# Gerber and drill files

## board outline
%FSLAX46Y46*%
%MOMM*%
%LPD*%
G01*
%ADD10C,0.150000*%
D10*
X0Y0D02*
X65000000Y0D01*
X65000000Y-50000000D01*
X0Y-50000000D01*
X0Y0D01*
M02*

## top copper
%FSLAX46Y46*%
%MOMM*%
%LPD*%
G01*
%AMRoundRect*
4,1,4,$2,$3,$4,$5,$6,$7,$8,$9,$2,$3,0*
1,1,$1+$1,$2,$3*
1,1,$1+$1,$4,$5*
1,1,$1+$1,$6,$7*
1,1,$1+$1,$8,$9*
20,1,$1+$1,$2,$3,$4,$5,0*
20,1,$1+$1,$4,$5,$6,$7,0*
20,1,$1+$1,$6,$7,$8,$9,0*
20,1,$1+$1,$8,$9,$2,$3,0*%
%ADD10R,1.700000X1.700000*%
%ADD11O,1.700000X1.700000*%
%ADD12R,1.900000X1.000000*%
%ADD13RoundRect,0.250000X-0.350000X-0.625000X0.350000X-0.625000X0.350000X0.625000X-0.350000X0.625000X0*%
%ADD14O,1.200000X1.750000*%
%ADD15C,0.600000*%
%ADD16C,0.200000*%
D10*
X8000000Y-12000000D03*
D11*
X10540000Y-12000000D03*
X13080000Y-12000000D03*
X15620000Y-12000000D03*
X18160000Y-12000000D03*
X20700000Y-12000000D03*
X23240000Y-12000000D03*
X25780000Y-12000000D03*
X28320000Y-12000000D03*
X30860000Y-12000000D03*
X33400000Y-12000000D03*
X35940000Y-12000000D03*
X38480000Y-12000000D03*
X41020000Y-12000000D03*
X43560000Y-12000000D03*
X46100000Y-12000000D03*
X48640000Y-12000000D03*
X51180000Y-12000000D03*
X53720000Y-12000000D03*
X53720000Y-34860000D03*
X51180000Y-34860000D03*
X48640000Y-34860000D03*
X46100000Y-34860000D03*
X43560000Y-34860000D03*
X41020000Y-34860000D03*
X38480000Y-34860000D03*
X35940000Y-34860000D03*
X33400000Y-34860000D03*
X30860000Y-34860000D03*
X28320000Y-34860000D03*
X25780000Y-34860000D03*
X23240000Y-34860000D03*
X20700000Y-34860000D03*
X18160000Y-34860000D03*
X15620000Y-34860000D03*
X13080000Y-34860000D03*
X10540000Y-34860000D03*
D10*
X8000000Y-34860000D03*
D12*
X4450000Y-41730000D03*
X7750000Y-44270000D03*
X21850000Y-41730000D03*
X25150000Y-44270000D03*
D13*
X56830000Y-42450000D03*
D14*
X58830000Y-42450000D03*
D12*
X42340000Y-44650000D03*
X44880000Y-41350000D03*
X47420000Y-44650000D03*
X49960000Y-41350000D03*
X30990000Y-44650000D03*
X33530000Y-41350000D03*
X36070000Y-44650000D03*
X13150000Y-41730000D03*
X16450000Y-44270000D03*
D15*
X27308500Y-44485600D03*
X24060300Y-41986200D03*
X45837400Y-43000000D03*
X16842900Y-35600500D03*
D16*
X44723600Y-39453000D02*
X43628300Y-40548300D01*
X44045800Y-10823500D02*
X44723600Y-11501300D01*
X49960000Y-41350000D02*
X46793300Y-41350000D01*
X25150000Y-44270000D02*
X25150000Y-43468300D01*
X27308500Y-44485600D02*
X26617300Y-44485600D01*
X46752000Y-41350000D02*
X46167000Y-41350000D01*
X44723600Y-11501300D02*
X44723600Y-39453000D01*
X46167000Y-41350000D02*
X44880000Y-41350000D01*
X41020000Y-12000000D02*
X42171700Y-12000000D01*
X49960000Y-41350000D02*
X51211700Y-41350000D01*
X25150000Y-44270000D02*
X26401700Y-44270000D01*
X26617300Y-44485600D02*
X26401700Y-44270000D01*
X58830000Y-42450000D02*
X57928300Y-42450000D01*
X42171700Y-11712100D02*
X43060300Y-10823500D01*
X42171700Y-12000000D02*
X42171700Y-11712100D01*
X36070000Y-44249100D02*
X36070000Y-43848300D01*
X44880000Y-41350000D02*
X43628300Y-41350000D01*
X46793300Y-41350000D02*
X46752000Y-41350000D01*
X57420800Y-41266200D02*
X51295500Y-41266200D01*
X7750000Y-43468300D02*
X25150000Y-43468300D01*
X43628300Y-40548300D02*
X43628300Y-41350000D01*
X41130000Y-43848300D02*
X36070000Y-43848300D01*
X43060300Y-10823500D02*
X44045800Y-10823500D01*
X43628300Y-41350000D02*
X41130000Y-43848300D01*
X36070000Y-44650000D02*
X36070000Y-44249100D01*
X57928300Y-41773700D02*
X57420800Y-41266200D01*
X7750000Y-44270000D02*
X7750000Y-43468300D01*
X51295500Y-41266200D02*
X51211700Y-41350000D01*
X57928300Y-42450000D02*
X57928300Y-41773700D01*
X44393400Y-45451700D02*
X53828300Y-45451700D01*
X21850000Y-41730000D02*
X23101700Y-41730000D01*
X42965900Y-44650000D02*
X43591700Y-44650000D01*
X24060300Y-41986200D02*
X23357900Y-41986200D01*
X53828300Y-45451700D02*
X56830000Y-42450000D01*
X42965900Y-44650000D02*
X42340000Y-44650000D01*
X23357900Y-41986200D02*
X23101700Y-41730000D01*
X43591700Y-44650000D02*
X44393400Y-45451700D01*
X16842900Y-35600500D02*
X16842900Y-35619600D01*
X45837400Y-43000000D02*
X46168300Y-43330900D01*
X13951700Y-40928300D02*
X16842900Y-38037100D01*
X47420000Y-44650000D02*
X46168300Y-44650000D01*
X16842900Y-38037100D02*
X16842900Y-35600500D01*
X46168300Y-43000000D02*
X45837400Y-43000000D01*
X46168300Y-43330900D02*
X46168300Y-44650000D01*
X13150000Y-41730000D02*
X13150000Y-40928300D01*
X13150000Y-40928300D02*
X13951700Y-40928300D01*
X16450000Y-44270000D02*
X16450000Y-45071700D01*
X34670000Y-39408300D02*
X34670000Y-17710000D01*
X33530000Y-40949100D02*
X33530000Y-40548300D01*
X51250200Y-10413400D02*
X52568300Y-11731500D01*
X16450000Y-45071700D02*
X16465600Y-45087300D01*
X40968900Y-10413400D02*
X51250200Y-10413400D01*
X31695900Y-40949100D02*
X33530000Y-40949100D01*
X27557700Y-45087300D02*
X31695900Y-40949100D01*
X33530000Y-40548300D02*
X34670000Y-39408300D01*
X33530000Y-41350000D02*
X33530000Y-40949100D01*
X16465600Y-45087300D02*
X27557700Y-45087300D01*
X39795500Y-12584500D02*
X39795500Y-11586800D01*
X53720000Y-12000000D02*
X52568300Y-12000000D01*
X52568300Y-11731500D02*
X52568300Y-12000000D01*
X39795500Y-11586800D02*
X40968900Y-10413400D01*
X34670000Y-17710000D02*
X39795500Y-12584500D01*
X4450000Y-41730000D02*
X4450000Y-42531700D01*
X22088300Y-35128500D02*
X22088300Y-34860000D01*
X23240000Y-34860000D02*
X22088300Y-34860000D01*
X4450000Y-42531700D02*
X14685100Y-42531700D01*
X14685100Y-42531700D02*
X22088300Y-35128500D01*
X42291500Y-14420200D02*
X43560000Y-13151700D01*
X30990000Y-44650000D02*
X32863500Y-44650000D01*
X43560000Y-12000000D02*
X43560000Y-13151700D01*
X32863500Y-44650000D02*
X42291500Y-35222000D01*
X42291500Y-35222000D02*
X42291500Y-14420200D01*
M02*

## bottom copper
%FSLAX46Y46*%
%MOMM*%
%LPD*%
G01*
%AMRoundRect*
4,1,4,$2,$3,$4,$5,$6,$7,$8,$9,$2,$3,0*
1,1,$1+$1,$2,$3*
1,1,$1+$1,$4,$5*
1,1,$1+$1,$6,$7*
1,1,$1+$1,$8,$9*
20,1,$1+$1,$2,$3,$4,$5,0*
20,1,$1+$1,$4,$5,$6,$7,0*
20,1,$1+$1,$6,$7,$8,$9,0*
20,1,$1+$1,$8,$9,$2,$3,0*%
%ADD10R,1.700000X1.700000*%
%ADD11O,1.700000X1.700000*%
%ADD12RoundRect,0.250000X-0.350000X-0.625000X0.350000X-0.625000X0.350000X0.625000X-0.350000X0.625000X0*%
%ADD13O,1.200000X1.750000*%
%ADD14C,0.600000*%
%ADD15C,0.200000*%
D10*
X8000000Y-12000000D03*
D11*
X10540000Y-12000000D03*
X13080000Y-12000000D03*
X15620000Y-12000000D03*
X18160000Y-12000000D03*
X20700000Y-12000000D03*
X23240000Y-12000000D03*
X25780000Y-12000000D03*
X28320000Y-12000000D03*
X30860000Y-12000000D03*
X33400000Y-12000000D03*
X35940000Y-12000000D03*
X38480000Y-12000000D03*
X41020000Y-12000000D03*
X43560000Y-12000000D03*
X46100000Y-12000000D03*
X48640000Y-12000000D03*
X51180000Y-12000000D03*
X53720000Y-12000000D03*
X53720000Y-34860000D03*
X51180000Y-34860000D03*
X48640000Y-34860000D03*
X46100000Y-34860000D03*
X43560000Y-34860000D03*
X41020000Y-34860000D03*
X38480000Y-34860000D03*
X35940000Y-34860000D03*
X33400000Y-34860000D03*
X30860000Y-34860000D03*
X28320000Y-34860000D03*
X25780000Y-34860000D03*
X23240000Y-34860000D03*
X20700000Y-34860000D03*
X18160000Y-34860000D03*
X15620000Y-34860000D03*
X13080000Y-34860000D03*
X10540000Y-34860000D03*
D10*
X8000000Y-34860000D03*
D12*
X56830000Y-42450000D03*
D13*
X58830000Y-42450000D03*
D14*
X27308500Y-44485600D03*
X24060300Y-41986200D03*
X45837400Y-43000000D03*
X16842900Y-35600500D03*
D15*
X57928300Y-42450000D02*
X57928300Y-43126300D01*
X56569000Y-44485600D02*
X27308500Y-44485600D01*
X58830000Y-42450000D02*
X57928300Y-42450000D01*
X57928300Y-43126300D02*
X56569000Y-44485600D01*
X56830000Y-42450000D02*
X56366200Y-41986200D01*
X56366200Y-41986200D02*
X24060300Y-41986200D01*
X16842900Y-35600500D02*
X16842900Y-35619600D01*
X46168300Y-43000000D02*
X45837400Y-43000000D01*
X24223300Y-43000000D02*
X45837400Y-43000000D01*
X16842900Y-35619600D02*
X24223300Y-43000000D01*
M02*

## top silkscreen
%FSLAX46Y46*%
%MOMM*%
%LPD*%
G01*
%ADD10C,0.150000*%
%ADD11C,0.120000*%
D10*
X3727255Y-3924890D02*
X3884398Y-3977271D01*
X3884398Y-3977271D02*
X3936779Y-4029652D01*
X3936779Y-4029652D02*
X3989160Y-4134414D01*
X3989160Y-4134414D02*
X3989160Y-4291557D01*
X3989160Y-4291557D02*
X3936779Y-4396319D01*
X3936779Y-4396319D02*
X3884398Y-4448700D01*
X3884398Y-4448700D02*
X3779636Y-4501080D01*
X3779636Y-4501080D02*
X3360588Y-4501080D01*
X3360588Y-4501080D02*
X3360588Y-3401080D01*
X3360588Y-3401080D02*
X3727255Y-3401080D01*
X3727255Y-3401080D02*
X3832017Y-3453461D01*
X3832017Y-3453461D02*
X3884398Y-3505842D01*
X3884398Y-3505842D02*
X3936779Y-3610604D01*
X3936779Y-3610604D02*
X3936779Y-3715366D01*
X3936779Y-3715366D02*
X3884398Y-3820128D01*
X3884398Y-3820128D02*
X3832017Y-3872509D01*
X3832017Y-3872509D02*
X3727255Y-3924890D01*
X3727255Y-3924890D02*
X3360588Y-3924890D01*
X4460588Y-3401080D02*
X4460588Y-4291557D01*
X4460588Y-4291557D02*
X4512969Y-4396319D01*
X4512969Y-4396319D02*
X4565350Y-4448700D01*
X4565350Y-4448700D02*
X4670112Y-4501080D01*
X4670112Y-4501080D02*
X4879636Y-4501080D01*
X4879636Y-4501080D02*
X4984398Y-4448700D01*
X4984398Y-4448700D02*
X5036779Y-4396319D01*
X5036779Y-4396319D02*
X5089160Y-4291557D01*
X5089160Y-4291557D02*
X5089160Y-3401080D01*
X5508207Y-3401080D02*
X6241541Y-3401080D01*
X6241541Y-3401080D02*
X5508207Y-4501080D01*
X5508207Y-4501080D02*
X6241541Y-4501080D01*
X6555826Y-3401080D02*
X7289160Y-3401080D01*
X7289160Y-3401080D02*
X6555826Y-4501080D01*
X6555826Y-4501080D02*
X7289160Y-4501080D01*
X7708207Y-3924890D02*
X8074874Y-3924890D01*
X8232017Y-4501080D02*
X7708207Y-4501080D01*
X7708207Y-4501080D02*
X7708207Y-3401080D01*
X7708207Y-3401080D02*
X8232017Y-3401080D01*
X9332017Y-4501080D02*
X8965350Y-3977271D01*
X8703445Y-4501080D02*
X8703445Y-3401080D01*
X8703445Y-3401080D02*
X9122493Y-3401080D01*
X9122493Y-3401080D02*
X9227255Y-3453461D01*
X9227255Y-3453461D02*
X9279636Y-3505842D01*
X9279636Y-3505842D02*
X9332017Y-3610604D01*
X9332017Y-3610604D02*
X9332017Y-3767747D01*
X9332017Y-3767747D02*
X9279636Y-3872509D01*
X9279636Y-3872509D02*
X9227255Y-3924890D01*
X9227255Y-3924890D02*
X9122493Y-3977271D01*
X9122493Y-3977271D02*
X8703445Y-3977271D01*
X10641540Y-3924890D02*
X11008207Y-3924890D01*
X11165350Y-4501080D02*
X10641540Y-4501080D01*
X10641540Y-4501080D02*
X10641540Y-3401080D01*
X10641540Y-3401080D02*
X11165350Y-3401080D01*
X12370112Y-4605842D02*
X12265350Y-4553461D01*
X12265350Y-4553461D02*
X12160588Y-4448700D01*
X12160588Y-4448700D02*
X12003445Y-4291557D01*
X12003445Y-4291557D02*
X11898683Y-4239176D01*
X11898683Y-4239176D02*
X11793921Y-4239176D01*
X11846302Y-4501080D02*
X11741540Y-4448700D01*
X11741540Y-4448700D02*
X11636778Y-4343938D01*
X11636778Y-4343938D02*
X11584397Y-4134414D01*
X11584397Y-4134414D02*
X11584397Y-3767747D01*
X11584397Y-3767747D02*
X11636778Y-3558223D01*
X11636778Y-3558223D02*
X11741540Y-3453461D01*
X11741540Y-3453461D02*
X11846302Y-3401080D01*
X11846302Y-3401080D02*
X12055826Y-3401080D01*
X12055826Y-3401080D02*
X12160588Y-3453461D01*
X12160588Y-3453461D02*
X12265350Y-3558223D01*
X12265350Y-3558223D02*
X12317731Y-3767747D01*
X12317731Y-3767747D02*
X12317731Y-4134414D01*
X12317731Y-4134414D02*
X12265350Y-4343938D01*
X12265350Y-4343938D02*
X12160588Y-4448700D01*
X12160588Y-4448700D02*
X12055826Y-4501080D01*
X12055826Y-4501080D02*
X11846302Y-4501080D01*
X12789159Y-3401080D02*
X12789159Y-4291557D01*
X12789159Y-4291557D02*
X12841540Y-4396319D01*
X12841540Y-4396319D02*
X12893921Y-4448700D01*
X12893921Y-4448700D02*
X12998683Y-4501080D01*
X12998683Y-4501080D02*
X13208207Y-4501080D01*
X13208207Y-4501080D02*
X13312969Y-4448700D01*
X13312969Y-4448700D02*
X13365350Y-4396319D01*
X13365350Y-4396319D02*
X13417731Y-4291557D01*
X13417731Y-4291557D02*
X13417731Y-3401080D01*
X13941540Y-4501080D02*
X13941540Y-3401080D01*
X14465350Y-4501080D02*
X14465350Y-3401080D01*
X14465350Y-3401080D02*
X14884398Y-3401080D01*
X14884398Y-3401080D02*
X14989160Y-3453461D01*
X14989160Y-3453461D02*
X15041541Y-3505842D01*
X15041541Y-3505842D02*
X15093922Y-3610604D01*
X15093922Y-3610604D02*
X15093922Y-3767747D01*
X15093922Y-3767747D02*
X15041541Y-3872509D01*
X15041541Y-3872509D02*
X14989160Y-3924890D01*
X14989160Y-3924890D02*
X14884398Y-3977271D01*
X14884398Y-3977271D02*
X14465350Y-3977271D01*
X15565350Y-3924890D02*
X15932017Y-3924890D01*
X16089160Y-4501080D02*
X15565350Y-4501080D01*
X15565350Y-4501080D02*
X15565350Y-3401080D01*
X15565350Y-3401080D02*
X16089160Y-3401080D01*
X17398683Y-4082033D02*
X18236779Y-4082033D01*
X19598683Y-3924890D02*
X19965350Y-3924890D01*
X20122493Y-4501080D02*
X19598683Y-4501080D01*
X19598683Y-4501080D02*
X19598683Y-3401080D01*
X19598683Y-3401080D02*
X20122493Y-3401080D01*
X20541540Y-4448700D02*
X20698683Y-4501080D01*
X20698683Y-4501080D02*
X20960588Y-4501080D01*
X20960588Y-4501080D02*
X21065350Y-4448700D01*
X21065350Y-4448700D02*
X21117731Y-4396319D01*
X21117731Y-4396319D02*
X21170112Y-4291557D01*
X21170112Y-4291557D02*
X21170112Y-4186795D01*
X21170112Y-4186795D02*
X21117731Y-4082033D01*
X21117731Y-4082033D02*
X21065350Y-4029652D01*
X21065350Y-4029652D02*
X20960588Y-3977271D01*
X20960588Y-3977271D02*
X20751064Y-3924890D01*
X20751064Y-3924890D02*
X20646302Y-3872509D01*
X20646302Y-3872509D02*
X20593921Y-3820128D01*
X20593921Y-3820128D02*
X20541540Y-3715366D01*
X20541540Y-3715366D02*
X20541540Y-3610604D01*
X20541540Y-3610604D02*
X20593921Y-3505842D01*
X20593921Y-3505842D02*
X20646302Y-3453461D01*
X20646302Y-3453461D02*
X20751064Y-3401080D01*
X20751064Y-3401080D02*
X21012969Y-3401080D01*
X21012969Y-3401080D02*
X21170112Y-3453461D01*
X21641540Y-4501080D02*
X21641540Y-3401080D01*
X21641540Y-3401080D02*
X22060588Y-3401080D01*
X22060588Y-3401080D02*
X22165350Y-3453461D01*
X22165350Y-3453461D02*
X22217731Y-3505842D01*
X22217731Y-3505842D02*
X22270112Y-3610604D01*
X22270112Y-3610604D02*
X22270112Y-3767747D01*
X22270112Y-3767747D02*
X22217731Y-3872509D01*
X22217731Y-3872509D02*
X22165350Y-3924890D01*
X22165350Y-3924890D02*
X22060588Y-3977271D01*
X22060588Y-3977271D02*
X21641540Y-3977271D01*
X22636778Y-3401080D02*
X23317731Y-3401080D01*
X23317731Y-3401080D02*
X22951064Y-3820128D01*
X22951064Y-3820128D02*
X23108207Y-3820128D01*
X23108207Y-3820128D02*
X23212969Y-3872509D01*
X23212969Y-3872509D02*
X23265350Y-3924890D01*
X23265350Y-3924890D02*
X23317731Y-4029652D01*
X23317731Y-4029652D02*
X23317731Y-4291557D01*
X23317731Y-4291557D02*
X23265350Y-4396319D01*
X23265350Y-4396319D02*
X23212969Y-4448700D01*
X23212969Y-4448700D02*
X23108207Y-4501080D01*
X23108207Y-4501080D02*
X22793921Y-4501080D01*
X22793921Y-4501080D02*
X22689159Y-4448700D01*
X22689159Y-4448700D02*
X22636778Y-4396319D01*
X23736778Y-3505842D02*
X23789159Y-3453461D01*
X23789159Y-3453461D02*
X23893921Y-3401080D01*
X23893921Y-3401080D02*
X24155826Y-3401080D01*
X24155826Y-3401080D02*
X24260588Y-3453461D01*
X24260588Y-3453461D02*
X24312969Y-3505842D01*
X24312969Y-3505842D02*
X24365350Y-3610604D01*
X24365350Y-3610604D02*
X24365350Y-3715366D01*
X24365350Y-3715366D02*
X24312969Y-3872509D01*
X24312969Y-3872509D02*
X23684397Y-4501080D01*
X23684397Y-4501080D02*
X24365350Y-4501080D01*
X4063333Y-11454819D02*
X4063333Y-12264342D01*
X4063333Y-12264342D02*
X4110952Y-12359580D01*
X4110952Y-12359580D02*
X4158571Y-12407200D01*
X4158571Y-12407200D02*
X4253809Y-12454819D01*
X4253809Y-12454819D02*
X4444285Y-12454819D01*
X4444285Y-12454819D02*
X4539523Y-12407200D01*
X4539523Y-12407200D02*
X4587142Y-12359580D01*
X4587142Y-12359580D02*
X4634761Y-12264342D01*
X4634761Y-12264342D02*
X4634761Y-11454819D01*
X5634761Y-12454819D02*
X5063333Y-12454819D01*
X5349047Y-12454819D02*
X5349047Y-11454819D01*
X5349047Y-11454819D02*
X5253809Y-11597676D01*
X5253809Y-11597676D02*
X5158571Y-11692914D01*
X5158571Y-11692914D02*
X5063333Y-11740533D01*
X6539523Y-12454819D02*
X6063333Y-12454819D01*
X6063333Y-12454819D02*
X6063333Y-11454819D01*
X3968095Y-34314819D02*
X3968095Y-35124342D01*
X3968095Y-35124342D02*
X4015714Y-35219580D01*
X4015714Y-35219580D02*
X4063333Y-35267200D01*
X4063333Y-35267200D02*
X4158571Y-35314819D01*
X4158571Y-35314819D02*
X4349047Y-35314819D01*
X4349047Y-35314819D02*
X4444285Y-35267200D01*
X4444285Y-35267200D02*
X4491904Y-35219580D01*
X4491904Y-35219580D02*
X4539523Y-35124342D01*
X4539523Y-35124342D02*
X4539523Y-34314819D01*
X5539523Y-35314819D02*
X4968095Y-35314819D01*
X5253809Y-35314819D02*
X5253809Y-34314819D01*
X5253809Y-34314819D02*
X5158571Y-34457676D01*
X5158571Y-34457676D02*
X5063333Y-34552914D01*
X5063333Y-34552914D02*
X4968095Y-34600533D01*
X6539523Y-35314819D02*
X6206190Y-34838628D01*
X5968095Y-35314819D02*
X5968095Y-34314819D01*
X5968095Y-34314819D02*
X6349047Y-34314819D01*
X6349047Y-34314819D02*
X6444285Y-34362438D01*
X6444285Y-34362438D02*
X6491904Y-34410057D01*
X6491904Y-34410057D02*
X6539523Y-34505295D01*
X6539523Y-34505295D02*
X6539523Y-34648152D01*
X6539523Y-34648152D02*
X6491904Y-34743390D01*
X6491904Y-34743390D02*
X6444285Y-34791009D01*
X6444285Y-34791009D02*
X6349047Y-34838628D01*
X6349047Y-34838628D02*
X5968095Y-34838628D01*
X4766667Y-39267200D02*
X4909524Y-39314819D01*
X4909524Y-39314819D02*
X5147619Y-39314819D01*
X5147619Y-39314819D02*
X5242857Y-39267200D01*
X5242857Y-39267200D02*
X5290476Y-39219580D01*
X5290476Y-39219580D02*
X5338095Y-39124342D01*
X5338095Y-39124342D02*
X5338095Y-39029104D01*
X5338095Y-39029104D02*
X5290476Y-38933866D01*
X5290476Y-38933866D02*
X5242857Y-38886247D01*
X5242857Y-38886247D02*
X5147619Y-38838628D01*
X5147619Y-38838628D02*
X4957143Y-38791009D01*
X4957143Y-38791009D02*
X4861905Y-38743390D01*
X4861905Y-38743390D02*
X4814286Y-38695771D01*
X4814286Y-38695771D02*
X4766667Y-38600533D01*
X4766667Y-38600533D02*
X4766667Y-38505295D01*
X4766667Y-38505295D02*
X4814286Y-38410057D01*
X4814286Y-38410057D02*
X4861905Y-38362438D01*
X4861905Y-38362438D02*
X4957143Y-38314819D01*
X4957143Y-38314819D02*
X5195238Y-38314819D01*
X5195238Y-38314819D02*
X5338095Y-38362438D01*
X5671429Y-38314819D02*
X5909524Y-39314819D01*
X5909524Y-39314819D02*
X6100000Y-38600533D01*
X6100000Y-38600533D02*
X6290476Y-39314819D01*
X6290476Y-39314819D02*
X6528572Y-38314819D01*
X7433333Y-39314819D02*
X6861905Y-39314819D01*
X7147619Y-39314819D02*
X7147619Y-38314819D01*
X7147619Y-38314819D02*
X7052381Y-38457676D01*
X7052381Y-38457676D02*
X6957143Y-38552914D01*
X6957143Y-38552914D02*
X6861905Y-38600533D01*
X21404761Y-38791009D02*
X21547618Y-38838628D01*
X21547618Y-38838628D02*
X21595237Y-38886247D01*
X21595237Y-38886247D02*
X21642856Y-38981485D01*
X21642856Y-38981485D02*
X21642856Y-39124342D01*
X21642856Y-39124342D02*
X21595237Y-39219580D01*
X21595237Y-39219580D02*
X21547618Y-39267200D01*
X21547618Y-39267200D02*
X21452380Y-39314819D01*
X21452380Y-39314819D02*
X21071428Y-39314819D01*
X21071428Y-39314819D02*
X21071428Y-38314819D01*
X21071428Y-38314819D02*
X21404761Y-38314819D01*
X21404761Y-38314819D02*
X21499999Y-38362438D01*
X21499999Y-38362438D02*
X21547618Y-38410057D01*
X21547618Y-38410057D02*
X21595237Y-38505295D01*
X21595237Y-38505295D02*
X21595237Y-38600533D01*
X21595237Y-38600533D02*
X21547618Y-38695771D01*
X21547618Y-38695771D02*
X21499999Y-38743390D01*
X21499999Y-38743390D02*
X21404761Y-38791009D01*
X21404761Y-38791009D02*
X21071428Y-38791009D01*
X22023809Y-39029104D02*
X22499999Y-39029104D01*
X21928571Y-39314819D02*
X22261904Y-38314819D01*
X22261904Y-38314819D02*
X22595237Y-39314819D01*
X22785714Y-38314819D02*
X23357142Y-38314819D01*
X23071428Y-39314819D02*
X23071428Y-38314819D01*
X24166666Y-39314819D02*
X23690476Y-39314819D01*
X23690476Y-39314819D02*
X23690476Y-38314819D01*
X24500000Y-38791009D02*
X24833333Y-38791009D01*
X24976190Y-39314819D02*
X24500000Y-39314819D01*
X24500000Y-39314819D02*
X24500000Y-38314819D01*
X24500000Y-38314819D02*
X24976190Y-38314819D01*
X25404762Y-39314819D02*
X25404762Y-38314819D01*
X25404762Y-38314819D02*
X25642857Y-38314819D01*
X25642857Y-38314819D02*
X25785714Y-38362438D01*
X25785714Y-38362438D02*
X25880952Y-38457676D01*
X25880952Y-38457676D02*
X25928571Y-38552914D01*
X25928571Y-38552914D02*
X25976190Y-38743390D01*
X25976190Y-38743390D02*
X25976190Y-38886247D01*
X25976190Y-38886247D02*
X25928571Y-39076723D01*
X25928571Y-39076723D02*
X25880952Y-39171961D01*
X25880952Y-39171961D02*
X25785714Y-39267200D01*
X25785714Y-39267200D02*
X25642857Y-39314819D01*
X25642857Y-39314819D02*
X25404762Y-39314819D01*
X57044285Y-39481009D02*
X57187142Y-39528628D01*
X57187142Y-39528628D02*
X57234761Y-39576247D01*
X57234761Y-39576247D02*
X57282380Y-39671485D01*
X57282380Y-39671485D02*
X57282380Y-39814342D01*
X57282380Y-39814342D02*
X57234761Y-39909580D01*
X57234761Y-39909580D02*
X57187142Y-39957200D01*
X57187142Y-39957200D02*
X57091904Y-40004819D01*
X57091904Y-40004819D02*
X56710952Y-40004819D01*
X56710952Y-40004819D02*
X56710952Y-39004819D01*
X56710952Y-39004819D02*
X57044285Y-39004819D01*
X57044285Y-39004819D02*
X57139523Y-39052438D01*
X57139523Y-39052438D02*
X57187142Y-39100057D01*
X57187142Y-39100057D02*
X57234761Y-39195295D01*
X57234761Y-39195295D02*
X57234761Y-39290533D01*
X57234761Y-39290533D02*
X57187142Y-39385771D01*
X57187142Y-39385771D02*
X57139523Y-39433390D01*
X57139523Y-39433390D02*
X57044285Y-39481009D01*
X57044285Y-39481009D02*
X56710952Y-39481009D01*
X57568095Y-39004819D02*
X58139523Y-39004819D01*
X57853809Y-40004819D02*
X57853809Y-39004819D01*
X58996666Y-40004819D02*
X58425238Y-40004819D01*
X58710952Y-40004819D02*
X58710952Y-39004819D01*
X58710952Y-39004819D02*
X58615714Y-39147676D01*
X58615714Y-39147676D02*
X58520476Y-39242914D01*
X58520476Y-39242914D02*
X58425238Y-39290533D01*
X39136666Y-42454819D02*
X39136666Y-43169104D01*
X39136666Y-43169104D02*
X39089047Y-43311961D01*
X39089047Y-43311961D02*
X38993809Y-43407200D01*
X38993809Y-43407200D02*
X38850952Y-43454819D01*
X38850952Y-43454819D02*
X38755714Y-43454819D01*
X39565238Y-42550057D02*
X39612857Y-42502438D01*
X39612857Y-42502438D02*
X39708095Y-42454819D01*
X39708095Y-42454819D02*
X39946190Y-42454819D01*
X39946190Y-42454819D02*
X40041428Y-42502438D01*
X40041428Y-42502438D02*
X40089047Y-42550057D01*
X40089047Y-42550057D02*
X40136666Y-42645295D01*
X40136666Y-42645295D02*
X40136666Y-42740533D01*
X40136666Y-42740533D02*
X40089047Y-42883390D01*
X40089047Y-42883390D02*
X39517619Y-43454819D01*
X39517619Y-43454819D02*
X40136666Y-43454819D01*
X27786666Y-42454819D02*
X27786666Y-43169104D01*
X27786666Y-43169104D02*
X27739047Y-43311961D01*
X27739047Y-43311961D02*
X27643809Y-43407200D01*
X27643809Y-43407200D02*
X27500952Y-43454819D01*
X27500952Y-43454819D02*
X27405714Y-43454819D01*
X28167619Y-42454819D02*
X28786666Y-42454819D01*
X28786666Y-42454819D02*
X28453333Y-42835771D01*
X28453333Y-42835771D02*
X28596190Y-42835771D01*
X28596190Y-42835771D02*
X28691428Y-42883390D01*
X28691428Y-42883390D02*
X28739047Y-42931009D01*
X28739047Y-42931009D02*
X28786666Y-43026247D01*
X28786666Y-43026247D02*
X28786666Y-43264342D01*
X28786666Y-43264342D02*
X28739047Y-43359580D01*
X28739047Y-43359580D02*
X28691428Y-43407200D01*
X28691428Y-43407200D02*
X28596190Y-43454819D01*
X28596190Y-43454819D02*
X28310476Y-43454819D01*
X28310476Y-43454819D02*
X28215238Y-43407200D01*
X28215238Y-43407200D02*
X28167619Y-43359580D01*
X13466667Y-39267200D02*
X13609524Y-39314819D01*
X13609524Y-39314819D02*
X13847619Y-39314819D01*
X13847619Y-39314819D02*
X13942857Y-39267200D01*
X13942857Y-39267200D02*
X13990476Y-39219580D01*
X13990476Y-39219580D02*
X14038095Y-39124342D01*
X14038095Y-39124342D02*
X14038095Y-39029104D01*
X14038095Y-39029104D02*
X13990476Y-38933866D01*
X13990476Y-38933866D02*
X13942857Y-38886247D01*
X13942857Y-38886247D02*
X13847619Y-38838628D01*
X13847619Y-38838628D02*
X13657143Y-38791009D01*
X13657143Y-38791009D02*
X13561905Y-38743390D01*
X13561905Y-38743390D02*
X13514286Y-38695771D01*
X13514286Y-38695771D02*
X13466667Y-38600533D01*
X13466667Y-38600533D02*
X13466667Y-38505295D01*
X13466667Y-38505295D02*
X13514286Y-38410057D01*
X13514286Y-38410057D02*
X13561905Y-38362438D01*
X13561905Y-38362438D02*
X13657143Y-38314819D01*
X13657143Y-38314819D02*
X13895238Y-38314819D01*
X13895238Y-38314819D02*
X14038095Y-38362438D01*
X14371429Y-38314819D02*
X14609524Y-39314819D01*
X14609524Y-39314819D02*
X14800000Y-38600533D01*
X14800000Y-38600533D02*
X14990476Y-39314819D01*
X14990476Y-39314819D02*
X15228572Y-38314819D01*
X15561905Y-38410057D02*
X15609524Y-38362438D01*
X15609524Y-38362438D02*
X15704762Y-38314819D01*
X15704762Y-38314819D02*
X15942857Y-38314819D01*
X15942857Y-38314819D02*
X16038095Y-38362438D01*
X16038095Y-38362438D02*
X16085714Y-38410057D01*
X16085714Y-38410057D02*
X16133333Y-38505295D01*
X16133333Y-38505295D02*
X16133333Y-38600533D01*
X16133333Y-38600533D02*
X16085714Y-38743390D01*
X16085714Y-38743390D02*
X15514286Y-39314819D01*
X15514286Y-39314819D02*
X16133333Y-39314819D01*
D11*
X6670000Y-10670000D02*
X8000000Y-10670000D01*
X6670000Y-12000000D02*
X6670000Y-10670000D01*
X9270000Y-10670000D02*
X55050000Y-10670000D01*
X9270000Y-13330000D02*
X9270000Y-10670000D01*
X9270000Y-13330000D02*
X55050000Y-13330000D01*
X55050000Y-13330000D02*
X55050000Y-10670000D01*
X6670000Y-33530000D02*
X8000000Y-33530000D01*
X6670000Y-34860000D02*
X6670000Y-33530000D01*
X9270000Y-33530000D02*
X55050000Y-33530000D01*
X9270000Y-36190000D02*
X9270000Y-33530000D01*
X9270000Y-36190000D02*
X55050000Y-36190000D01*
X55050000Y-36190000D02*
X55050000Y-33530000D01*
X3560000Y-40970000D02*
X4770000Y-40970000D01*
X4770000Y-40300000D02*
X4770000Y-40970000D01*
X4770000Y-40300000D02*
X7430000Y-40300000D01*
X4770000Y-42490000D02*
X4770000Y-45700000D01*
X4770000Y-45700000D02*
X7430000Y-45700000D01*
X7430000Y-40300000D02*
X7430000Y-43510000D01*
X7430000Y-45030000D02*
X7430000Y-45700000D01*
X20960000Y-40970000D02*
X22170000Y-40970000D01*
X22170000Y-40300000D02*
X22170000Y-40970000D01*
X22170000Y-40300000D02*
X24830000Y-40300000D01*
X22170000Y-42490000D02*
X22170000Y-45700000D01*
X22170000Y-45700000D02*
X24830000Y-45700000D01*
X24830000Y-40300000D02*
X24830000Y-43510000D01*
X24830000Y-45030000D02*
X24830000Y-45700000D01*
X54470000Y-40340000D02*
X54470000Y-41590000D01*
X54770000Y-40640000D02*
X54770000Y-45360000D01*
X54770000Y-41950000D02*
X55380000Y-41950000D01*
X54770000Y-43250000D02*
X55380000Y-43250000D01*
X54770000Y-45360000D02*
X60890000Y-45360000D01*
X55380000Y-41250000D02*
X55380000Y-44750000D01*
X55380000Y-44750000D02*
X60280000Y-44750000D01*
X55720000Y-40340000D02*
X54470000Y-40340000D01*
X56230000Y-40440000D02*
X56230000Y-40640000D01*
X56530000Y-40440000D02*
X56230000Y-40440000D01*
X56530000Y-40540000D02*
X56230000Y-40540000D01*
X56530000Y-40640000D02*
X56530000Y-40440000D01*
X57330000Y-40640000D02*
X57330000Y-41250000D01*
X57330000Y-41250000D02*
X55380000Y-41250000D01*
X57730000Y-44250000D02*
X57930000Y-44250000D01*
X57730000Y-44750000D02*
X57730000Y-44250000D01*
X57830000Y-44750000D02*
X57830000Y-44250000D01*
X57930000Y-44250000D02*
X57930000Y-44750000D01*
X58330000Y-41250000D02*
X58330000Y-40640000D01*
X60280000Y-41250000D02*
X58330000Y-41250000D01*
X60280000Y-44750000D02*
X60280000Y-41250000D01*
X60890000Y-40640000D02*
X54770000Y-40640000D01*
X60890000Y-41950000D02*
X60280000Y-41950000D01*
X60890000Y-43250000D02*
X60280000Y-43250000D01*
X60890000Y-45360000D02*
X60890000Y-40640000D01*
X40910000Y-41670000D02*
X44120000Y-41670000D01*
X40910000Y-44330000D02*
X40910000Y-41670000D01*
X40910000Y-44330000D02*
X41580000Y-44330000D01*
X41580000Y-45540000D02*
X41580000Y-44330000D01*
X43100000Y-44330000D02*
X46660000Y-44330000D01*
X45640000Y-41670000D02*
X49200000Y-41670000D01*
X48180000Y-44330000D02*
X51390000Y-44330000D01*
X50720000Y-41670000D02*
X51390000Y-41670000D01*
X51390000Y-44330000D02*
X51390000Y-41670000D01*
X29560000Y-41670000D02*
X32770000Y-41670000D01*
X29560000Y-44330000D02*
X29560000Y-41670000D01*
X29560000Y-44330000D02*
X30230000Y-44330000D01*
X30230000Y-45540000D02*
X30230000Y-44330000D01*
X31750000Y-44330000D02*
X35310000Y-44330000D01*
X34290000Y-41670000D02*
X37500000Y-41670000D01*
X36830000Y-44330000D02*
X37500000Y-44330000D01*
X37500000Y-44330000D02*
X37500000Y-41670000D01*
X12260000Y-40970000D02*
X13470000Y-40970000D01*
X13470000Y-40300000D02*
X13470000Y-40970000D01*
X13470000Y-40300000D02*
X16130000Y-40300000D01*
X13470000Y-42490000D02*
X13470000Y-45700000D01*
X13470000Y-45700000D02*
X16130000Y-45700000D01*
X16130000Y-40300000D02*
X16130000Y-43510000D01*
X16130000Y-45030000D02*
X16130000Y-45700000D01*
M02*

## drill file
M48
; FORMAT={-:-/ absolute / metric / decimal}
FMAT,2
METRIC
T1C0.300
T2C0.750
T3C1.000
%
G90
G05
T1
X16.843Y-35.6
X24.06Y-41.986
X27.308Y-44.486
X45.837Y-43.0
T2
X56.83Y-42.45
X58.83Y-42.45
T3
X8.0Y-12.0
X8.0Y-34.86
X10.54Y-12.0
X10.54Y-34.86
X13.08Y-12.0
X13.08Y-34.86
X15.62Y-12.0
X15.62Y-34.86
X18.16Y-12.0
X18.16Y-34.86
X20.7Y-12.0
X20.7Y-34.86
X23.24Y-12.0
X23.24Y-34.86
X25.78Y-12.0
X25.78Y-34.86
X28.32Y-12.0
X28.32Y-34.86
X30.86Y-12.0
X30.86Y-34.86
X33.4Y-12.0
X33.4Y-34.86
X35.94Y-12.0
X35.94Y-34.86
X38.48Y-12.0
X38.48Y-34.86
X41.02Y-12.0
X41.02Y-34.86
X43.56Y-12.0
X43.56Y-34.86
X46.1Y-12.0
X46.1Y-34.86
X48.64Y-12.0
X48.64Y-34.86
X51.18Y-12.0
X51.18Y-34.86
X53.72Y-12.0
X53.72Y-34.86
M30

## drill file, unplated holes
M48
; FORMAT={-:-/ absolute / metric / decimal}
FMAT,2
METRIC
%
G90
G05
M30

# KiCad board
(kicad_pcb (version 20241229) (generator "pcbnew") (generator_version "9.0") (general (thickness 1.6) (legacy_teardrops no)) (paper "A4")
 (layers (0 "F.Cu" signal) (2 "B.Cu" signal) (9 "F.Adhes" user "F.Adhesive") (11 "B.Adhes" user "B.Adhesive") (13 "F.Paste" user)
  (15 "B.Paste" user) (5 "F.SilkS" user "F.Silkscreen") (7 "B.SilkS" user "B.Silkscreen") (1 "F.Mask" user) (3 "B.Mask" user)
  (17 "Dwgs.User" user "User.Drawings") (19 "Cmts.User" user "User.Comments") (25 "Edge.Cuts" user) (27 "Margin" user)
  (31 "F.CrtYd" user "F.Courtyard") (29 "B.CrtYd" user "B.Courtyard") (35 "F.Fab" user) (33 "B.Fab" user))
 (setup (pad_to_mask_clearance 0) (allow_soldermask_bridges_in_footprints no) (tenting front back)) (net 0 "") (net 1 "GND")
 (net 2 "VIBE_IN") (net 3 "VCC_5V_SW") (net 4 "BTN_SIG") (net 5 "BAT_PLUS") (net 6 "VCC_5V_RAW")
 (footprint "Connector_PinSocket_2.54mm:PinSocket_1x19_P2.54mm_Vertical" (layer "F.Cu") (at 8 12 90)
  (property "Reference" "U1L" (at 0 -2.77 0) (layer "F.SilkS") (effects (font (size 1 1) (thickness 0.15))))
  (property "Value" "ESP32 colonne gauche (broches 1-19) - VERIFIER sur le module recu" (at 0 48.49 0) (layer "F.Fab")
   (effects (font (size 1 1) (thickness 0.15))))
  (fp_line (start 1.33 -1.33) (end 1.33 0) (stroke (width 0.12) (type solid)) (layer "F.SilkS"))
  (fp_line (start 0 -1.33) (end 1.33 -1.33) (stroke (width 0.12) (type solid)) (layer "F.SilkS"))
  (fp_line (start 1.33 1.27) (end 1.33 47.05) (stroke (width 0.12) (type solid)) (layer "F.SilkS"))
  (fp_line (start -1.33 1.27) (end 1.33 1.27) (stroke (width 0.12) (type solid)) (layer "F.SilkS"))
  (fp_line (start -1.33 1.27) (end -1.33 47.05) (stroke (width 0.12) (type solid)) (layer "F.SilkS"))
  (fp_line (start -1.33 47.05) (end 1.33 47.05) (stroke (width 0.12) (type solid)) (layer "F.SilkS"))
  (pad "1" thru_hole rect (at 0 0) (size 1.7 1.7) (drill 1) (layers "*.Cu" "*.Mask") (remove_unused_layers no))
  (pad "2" thru_hole oval (at 0 2.54) (size 1.7 1.7) (drill 1) (layers "*.Cu" "*.Mask") (remove_unused_layers no))
  (pad "3" thru_hole oval (at 0 5.08) (size 1.7 1.7) (drill 1) (layers "*.Cu" "*.Mask") (remove_unused_layers no))
  (pad "4" thru_hole oval (at 0 7.62) (size 1.7 1.7) (drill 1) (layers "*.Cu" "*.Mask") (remove_unused_layers no))
  (pad "5" thru_hole oval (at 0 10.16) (size 1.7 1.7) (drill 1) (layers "*.Cu" "*.Mask") (remove_unused_layers no))
  (pad "6" thru_hole oval (at 0 12.7) (size 1.7 1.7) (drill 1) (layers "*.Cu" "*.Mask") (remove_unused_layers no))
  (pad "7" thru_hole oval (at 0 15.24) (size 1.7 1.7) (drill 1) (layers "*.Cu" "*.Mask") (remove_unused_layers no))
  (pad "8" thru_hole oval (at 0 17.78) (size 1.7 1.7) (drill 1) (layers "*.Cu" "*.Mask") (remove_unused_layers no))
  (pad "9" thru_hole oval (at 0 20.32) (size 1.7 1.7) (drill 1) (layers "*.Cu" "*.Mask") (remove_unused_layers no))
  (pad "10" thru_hole oval (at 0 22.86) (size 1.7 1.7) (drill 1) (layers "*.Cu" "*.Mask") (remove_unused_layers no))
  (pad "11" thru_hole oval (at 0 25.4) (size 1.7 1.7) (drill 1) (layers "*.Cu" "*.Mask") (remove_unused_layers no))
  (pad "12" thru_hole oval (at 0 27.94) (size 1.7 1.7) (drill 1) (layers "*.Cu" "*.Mask") (remove_unused_layers no))
  (pad "13" thru_hole oval (at 0 30.48) (size 1.7 1.7) (drill 1) (layers "*.Cu" "*.Mask") (remove_unused_layers no))
  (pad "14" thru_hole oval (at 0 33.02) (size 1.7 1.7) (drill 1) (layers "*.Cu" "*.Mask") (remove_unused_layers no) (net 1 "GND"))
  (pad "15" thru_hole oval (at 0 35.56) (size 1.7 1.7) (drill 1) (layers "*.Cu" "*.Mask") (remove_unused_layers no) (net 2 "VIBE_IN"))
  (pad "16" thru_hole oval (at 0 38.1) (size 1.7 1.7) (drill 1) (layers "*.Cu" "*.Mask") (remove_unused_layers no))
  (pad "17" thru_hole oval (at 0 40.64) (size 1.7 1.7) (drill 1) (layers "*.Cu" "*.Mask") (remove_unused_layers no))
  (pad "18" thru_hole oval (at 0 43.18) (size 1.7 1.7) (drill 1) (layers "*.Cu" "*.Mask") (remove_unused_layers no))
  (pad "19" thru_hole oval (at 0 45.72) (size 1.7 1.7) (drill 1) (layers "*.Cu" "*.Mask") (remove_unused_layers no) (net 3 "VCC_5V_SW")))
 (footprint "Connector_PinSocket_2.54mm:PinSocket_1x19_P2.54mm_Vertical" (layer "F.Cu") (at 8 34.86 90)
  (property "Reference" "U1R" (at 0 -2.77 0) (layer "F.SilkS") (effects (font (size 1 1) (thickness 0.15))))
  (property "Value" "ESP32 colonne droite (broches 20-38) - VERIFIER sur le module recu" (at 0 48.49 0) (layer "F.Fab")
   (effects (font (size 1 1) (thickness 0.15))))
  (fp_line (start 1.33 -1.33) (end 1.33 0) (stroke (width 0.12) (type solid)) (layer "F.SilkS"))
  (fp_line (start 0 -1.33) (end 1.33 -1.33) (stroke (width 0.12) (type solid)) (layer "F.SilkS"))
  (fp_line (start 1.33 1.27) (end 1.33 47.05) (stroke (width 0.12) (type solid)) (layer "F.SilkS"))
  (fp_line (start -1.33 1.27) (end 1.33 1.27) (stroke (width 0.12) (type solid)) (layer "F.SilkS"))
  (fp_line (start -1.33 1.27) (end -1.33 47.05) (stroke (width 0.12) (type solid)) (layer "F.SilkS"))
  (fp_line (start -1.33 47.05) (end 1.33 47.05) (stroke (width 0.12) (type solid)) (layer "F.SilkS"))
  (pad "20" thru_hole oval (at 0 45.72) (size 1.7 1.7) (drill 1) (layers "*.Cu" "*.Mask") (remove_unused_layers no))
  (pad "21" thru_hole oval (at 0 43.18) (size 1.7 1.7) (drill 1) (layers "*.Cu" "*.Mask") (remove_unused_layers no))
  (pad "22" thru_hole oval (at 0 40.64) (size 1.7 1.7) (drill 1) (layers "*.Cu" "*.Mask") (remove_unused_layers no))
  (pad "23" thru_hole oval (at 0 38.1) (size 1.7 1.7) (drill 1) (layers "*.Cu" "*.Mask") (remove_unused_layers no))
  (pad "24" thru_hole oval (at 0 35.56) (size 1.7 1.7) (drill 1) (layers "*.Cu" "*.Mask") (remove_unused_layers no))
  (pad "25" thru_hole oval (at 0 33.02) (size 1.7 1.7) (drill 1) (layers "*.Cu" "*.Mask") (remove_unused_layers no))
  (pad "26" thru_hole oval (at 0 30.48) (size 1.7 1.7) (drill 1) (layers "*.Cu" "*.Mask") (remove_unused_layers no))
  (pad "27" thru_hole oval (at 0 27.94) (size 1.7 1.7) (drill 1) (layers "*.Cu" "*.Mask") (remove_unused_layers no))
  (pad "28" thru_hole oval (at 0 25.4) (size 1.7 1.7) (drill 1) (layers "*.Cu" "*.Mask") (remove_unused_layers no))
  (pad "29" thru_hole oval (at 0 22.86) (size 1.7 1.7) (drill 1) (layers "*.Cu" "*.Mask") (remove_unused_layers no))
  (pad "30" thru_hole oval (at 0 20.32) (size 1.7 1.7) (drill 1) (layers "*.Cu" "*.Mask") (remove_unused_layers no))
  (pad "31" thru_hole oval (at 0 17.78) (size 1.7 1.7) (drill 1) (layers "*.Cu" "*.Mask") (remove_unused_layers no))
  (pad "32" thru_hole oval (at 0 15.24) (size 1.7 1.7) (drill 1) (layers "*.Cu" "*.Mask") (remove_unused_layers no) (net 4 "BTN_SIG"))
  (pad "33" thru_hole oval (at 0 12.7) (size 1.7 1.7) (drill 1) (layers "*.Cu" "*.Mask") (remove_unused_layers no))
  (pad "34" thru_hole oval (at 0 10.16) (size 1.7 1.7) (drill 1) (layers "*.Cu" "*.Mask") (remove_unused_layers no))
  (pad "35" thru_hole oval (at 0 7.62) (size 1.7 1.7) (drill 1) (layers "*.Cu" "*.Mask") (remove_unused_layers no))
  (pad "36" thru_hole oval (at 0 5.08) (size 1.7 1.7) (drill 1) (layers "*.Cu" "*.Mask") (remove_unused_layers no))
  (pad "37" thru_hole oval (at 0 2.54) (size 1.7 1.7) (drill 1) (layers "*.Cu" "*.Mask") (remove_unused_layers no))
  (pad "38" thru_hole rect (at 0 0) (size 1.7 1.7) (drill 1) (layers "*.Cu" "*.Mask") (remove_unused_layers no)))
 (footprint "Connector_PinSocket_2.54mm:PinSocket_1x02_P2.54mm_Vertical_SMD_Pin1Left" (layer "F.Cu") (at 6.1 43)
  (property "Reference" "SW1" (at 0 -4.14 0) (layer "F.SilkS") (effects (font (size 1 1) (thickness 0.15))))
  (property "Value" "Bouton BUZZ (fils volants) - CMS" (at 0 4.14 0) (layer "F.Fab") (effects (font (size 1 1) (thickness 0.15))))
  (fp_line (start -2.54 -2.03) (end -1.33 -2.03) (stroke (width 0.12) (type solid)) (layer "F.SilkS"))
  (fp_line (start -1.33 -2.7) (end -1.33 -2.03) (stroke (width 0.12) (type solid)) (layer "F.SilkS"))
  (fp_line (start -1.33 -2.7) (end 1.33 -2.7) (stroke (width 0.12) (type solid)) (layer "F.SilkS"))
  (fp_line (start -1.33 -0.51) (end -1.33 2.7) (stroke (width 0.12) (type solid)) (layer "F.SilkS"))
  (fp_line (start -1.33 2.7) (end 1.33 2.7) (stroke (width 0.12) (type solid)) (layer "F.SilkS"))
  (fp_line (start 1.33 -2.7) (end 1.33 0.51) (stroke (width 0.12) (type solid)) (layer "F.SilkS"))
  (fp_line (start 1.33 2.03) (end 1.33 2.7) (stroke (width 0.12) (type solid)) (layer "F.SilkS"))
  (pad "1" smd rect (at -1.65 -1.27) (size 1.9 1) (layers "F.Cu" "F.Mask" "F.Paste") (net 4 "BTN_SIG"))
  (pad "2" smd rect (at 1.65 1.27) (size 1.9 1) (layers "F.Cu" "F.Mask" "F.Paste") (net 1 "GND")))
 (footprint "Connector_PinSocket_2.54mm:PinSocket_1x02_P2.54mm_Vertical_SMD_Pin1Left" (layer "F.Cu") (at 23.5 43)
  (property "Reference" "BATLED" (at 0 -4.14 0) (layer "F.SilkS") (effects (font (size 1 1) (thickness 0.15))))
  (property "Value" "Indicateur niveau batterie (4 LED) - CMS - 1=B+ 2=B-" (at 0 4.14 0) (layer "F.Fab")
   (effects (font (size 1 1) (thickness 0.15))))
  (fp_line (start -2.54 -2.03) (end -1.33 -2.03) (stroke (width 0.12) (type solid)) (layer "F.SilkS"))
  (fp_line (start -1.33 -2.7) (end -1.33 -2.03) (stroke (width 0.12) (type solid)) (layer "F.SilkS"))
  (fp_line (start -1.33 -2.7) (end 1.33 -2.7) (stroke (width 0.12) (type solid)) (layer "F.SilkS"))
  (fp_line (start -1.33 -0.51) (end -1.33 2.7) (stroke (width 0.12) (type solid)) (layer "F.SilkS"))
  (fp_line (start -1.33 2.7) (end 1.33 2.7) (stroke (width 0.12) (type solid)) (layer "F.SilkS"))
  (fp_line (start 1.33 -2.7) (end 1.33 0.51) (stroke (width 0.12) (type solid)) (layer "F.SilkS"))
  (fp_line (start 1.33 2.03) (end 1.33 2.7) (stroke (width 0.12) (type solid)) (layer "F.SilkS"))
  (pad "1" smd rect (at -1.65 -1.27) (size 1.9 1) (layers "F.Cu" "F.Mask" "F.Paste") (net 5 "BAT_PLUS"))
  (pad "2" smd rect (at 1.65 1.27) (size 1.9 1) (layers "F.Cu" "F.Mask" "F.Paste") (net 1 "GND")))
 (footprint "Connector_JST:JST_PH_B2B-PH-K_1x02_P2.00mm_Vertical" (layer "F.Cu") (at 56.83 42.45)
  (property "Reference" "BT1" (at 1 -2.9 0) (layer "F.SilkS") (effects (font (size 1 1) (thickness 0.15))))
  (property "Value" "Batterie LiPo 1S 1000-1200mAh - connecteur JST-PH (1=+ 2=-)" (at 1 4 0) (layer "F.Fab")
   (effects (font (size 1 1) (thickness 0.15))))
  (fp_line (start -2.36 -2.11) (end -2.36 -0.86) (stroke (width 0.12) (type solid)) (layer "F.SilkS"))
  (fp_line (start -2.06 -1.81) (end -2.06 2.91) (stroke (width 0.12) (type solid)) (layer "F.SilkS"))
  (fp_line (start -2.06 -0.5) (end -1.45 -0.5) (stroke (width 0.12) (type solid)) (layer "F.SilkS"))
  (fp_line (start -2.06 0.8) (end -1.45 0.8) (stroke (width 0.12) (type solid)) (layer "F.SilkS"))
  (fp_line (start -2.06 2.91) (end 4.06 2.91) (stroke (width 0.12) (type solid)) (layer "F.SilkS"))
  (fp_line (start -1.45 -1.2) (end -1.45 2.3) (stroke (width 0.12) (type solid)) (layer "F.SilkS"))
  (fp_line (start -1.45 2.3) (end 3.45 2.3) (stroke (width 0.12) (type solid)) (layer "F.SilkS"))
  (fp_line (start -1.11 -2.11) (end -2.36 -2.11) (stroke (width 0.12) (type solid)) (layer "F.SilkS"))
  (fp_line (start -0.6 -2.01) (end -0.6 -1.81) (stroke (width 0.12) (type solid)) (layer "F.SilkS"))
  (fp_line (start -0.3 -2.01) (end -0.6 -2.01) (stroke (width 0.12) (type solid)) (layer "F.SilkS"))
  (fp_line (start -0.3 -1.91) (end -0.6 -1.91) (stroke (width 0.12) (type solid)) (layer "F.SilkS"))
  (fp_line (start -0.3 -1.81) (end -0.3 -2.01) (stroke (width 0.12) (type solid)) (layer "F.SilkS"))
  (fp_line (start 0.5 -1.81) (end 0.5 -1.2) (stroke (width 0.12) (type solid)) (layer "F.SilkS"))
  (fp_line (start 0.5 -1.2) (end -1.45 -1.2) (stroke (width 0.12) (type solid)) (layer "F.SilkS"))
  (fp_line (start 0.9 1.8) (end 1.1 1.8) (stroke (width 0.12) (type solid)) (layer "F.SilkS"))
  (fp_line (start 0.9 2.3) (end 0.9 1.8) (stroke (width 0.12) (type solid)) (layer "F.SilkS"))
  (fp_line (start 1 2.3) (end 1 1.8) (stroke (width 0.12) (type solid)) (layer "F.SilkS"))
  (fp_line (start 1.1 1.8) (end 1.1 2.3) (stroke (width 0.12) (type solid)) (layer "F.SilkS"))
  (fp_line (start 1.5 -1.2) (end 1.5 -1.81) (stroke (width 0.12) (type solid)) (layer "F.SilkS"))
  (fp_line (start 3.45 -1.2) (end 1.5 -1.2) (stroke (width 0.12) (type solid)) (layer "F.SilkS"))
  (fp_line (start 3.45 2.3) (end 3.45 -1.2) (stroke (width 0.12) (type solid)) (layer "F.SilkS"))
  (fp_line (start 4.06 -1.81) (end -2.06 -1.81) (stroke (width 0.12) (type solid)) (layer "F.SilkS"))
  (fp_line (start 4.06 -0.5) (end 3.45 -0.5) (stroke (width 0.12) (type solid)) (layer "F.SilkS"))
  (fp_line (start 4.06 0.8) (end 3.45 0.8) (stroke (width 0.12) (type solid)) (layer "F.SilkS"))
  (fp_line (start 4.06 2.91) (end 4.06 -1.81) (stroke (width 0.12) (type solid)) (layer "F.SilkS"))
  (pad "1" thru_hole roundrect (at 0 0) (size 1.2 1.75) (drill 0.75) (layers "*.Cu" "*.Mask") (remove_unused_layers no)
   (roundrect_rratio 0.208333) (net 5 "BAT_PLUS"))
  (pad "2" thru_hole oval (at 2 0) (size 1.2 1.75) (drill 0.75) (layers "*.Cu" "*.Mask") (remove_unused_layers no) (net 1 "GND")))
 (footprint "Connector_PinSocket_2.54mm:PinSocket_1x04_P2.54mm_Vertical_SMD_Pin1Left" (layer "F.Cu") (at 46.15 43 90)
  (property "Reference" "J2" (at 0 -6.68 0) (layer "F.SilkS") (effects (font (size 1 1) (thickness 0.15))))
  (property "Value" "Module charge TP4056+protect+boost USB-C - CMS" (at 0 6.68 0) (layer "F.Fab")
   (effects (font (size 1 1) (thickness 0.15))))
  (fp_line (start 1.33 -5.24) (end 1.33 -2.03) (stroke (width 0.12) (type solid)) (layer "F.SilkS"))
  (fp_line (start -1.33 -5.24) (end 1.33 -5.24) (stroke (width 0.12) (type solid)) (layer "F.SilkS"))
  (fp_line (start -1.33 -5.24) (end -1.33 -4.57) (stroke (width 0.12) (type solid)) (layer "F.SilkS"))
  (fp_line (start -2.54 -4.57) (end -1.33 -4.57) (stroke (width 0.12) (type solid)) (layer "F.SilkS"))
  (fp_line (start -1.33 -3.05) (end -1.33 0.51) (stroke (width 0.12) (type solid)) (layer "F.SilkS"))
  (fp_line (start 1.33 -0.51) (end 1.33 3.05) (stroke (width 0.12) (type solid)) (layer "F.SilkS"))
  (fp_line (start -1.33 2.03) (end -1.33 5.24) (stroke (width 0.12) (type solid)) (layer "F.SilkS"))
  (fp_line (start 1.33 4.57) (end 1.33 5.24) (stroke (width 0.12) (type solid)) (layer "F.SilkS"))
  (fp_line (start -1.33 5.24) (end 1.33 5.24) (stroke (width 0.12) (type solid)) (layer "F.SilkS"))
  (pad "1" smd rect (at -1.65 -3.81) (size 1.9 1) (layers "F.Cu" "F.Mask" "F.Paste") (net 5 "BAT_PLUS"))
  (pad "2" smd rect (at 1.65 -1.27) (size 1.9 1) (layers "F.Cu" "F.Mask" "F.Paste") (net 1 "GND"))
  (pad "3" smd rect (at -1.65 1.27) (size 1.9 1) (layers "F.Cu" "F.Mask" "F.Paste") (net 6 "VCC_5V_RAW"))
  (pad "4" smd rect (at 1.65 3.81) (size 1.9 1) (layers "F.Cu" "F.Mask" "F.Paste") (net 1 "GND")))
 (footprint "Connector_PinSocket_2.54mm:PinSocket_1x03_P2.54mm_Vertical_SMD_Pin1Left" (layer "F.Cu") (at 33.53 43 90)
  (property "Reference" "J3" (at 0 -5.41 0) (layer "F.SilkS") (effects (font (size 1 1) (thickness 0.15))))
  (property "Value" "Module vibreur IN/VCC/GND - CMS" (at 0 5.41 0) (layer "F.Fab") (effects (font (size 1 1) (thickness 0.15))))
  (fp_line (start 1.33 -3.97) (end 1.33 -0.76) (stroke (width 0.12) (type solid)) (layer "F.SilkS"))
  (fp_line (start -1.33 -3.97) (end 1.33 -3.97) (stroke (width 0.12) (type solid)) (layer "F.SilkS"))
  (fp_line (start -1.33 -3.97) (end -1.33 -3.3) (stroke (width 0.12) (type solid)) (layer "F.SilkS"))
  (fp_line (start -2.54 -3.3) (end -1.33 -3.3) (stroke (width 0.12) (type solid)) (layer "F.SilkS"))
  (fp_line (start -1.33 -1.78) (end -1.33 1.78) (stroke (width 0.12) (type solid)) (layer "F.SilkS"))
  (fp_line (start 1.33 0.76) (end 1.33 3.97) (stroke (width 0.12) (type solid)) (layer "F.SilkS"))
  (fp_line (start -1.33 3.3) (end -1.33 3.97) (stroke (width 0.12) (type solid)) (layer "F.SilkS"))
  (fp_line (start -1.33 3.97) (end 1.33 3.97) (stroke (width 0.12) (type solid)) (layer "F.SilkS"))
  (pad "1" smd rect (at -1.65 -2.54) (size 1.9 1) (layers "F.Cu" "F.Mask" "F.Paste") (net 2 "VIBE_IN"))
  (pad "2" smd rect (at 1.65 0) (size 1.9 1) (layers "F.Cu" "F.Mask" "F.Paste") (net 3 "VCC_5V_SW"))
  (pad "3" smd rect (at -1.65 2.54) (size 1.9 1) (layers "F.Cu" "F.Mask" "F.Paste") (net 1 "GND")))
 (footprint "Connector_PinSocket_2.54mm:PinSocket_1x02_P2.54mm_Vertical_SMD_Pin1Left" (layer "F.Cu") (at 14.8 43)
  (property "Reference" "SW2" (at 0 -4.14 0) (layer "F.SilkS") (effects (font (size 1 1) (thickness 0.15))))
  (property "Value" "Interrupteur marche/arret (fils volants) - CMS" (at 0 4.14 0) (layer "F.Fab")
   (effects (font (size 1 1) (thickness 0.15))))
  (fp_line (start -2.54 -2.03) (end -1.33 -2.03) (stroke (width 0.12) (type solid)) (layer "F.SilkS"))
  (fp_line (start -1.33 -2.7) (end -1.33 -2.03) (stroke (width 0.12) (type solid)) (layer "F.SilkS"))
  (fp_line (start -1.33 -2.7) (end 1.33 -2.7) (stroke (width 0.12) (type solid)) (layer "F.SilkS"))
  (fp_line (start -1.33 -0.51) (end -1.33 2.7) (stroke (width 0.12) (type solid)) (layer "F.SilkS"))
  (fp_line (start -1.33 2.7) (end 1.33 2.7) (stroke (width 0.12) (type solid)) (layer "F.SilkS"))
  (fp_line (start 1.33 -2.7) (end 1.33 0.51) (stroke (width 0.12) (type solid)) (layer "F.SilkS"))
  (fp_line (start 1.33 2.03) (end 1.33 2.7) (stroke (width 0.12) (type solid)) (layer "F.SilkS"))
  (pad "1" smd rect (at -1.65 -1.27) (size 1.9 1) (layers "F.Cu" "F.Mask" "F.Paste") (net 6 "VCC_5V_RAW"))
  (pad "2" smd rect (at 1.65 1.27) (size 1.9 1) (layers "F.Cu" "F.Mask" "F.Paste") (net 3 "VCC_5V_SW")))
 (gr_rect (start 0 0) (end 65 50) (stroke (width 0.15) (type default)) (fill no) (layer "Edge.Cuts"))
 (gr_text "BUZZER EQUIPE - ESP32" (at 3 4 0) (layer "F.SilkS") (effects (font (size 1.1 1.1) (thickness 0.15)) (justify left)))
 (segment (start 44.7236 39.453) (end 43.6283 40.5483) (width 0.2) (layer "F.Cu") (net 1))
 (segment (start 44.0458 10.8235) (end 44.7236 11.5013) (width 0.2) (layer "F.Cu") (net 1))
 (segment (start 49.96 41.35) (end 46.7933 41.35) (width 0.2) (layer "F.Cu") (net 1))
 (segment (start 25.15 44.27) (end 25.15 43.4683) (width 0.2) (layer "F.Cu") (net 1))
 (segment (start 27.3085 44.4856) (end 26.6173 44.4856) (width 0.2) (layer "F.Cu") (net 1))
 (segment (start 46.752 41.35) (end 46.167 41.35) (width 0.2) (layer "F.Cu") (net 1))
 (segment (start 44.7236 11.5013) (end 44.7236 39.453) (width 0.2) (layer "F.Cu") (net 1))
 (segment (start 46.167 41.35) (end 44.88 41.35) (width 0.2) (layer "F.Cu") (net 1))
 (segment (start 41.02 12) (end 42.1717 12) (width 0.2) (layer "F.Cu") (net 1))
 (segment (start 49.96 41.35) (end 51.2117 41.35) (width 0.2) (layer "F.Cu") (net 1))
 (segment (start 25.15 44.27) (end 26.4017 44.27) (width 0.2) (layer "F.Cu") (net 1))
 (segment (start 26.6173 44.4856) (end 26.4017 44.27) (width 0.2) (layer "F.Cu") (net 1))
 (segment (start 58.83 42.45) (end 57.9283 42.45) (width 0.2) (layer "F.Cu") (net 1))
 (segment (start 42.1717 11.7121) (end 43.0603 10.8235) (width 0.2) (layer "F.Cu") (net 1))
 (segment (start 42.1717 12) (end 42.1717 11.7121) (width 0.2) (layer "F.Cu") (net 1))
 (segment (start 36.07 44.2491) (end 36.07 43.8483) (width 0.2) (layer "F.Cu") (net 1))
 (segment (start 44.88 41.35) (end 43.6283 41.35) (width 0.2) (layer "F.Cu") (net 1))
 (segment (start 46.7933 41.35) (end 46.752 41.35) (width 0.2) (layer "F.Cu") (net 1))
 (segment (start 57.4208 41.2662) (end 51.2955 41.2662) (width 0.2) (layer "F.Cu") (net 1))
 (segment (start 7.75 43.4683) (end 25.15 43.4683) (width 0.2) (layer "F.Cu") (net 1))
 (segment (start 43.6283 40.5483) (end 43.6283 41.35) (width 0.2) (layer "F.Cu") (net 1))
 (segment (start 41.13 43.8483) (end 36.07 43.8483) (width 0.2) (layer "F.Cu") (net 1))
 (segment (start 43.0603 10.8235) (end 44.0458 10.8235) (width 0.2) (layer "F.Cu") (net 1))
 (segment (start 43.6283 41.35) (end 41.13 43.8483) (width 0.2) (layer "F.Cu") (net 1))
 (segment (start 36.07 44.65) (end 36.07 44.2491) (width 0.2) (layer "F.Cu") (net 1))
 (segment (start 57.9283 41.7737) (end 57.4208 41.2662) (width 0.2) (layer "F.Cu") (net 1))
 (segment (start 7.75 44.27) (end 7.75 43.4683) (width 0.2) (layer "F.Cu") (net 1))
 (segment (start 51.2955 41.2662) (end 51.2117 41.35) (width 0.2) (layer "F.Cu") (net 1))
 (segment (start 57.9283 42.45) (end 57.9283 41.7737) (width 0.2) (layer "F.Cu") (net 1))
 (via (at 27.3085 44.4856) (size 0.6) (drill 0.3) (layers "F.Cu" "B.Cu") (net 1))
 (segment (start 57.9283 42.45) (end 57.9283 43.1263) (width 0.2) (layer "B.Cu") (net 1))
 (segment (start 56.569 44.4856) (end 27.3085 44.4856) (width 0.2) (layer "B.Cu") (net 1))
 (segment (start 58.83 42.45) (end 57.9283 42.45) (width 0.2) (layer "B.Cu") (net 1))
 (segment (start 57.9283 43.1263) (end 56.569 44.4856) (width 0.2) (layer "B.Cu") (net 1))
 (segment (start 44.3934 45.4517) (end 53.8283 45.4517) (width 0.2) (layer "F.Cu") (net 5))
 (segment (start 21.85 41.73) (end 23.1017 41.73) (width 0.2) (layer "F.Cu") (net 5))
 (segment (start 42.9659 44.65) (end 43.5917 44.65) (width 0.2) (layer "F.Cu") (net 5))
 (segment (start 24.0603 41.9862) (end 23.3579 41.9862) (width 0.2) (layer "F.Cu") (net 5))
 (segment (start 53.8283 45.4517) (end 56.83 42.45) (width 0.2) (layer "F.Cu") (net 5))
 (segment (start 42.9659 44.65) (end 42.34 44.65) (width 0.2) (layer "F.Cu") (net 5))
 (segment (start 23.3579 41.9862) (end 23.1017 41.73) (width 0.2) (layer "F.Cu") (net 5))
 (segment (start 43.5917 44.65) (end 44.3934 45.4517) (width 0.2) (layer "F.Cu") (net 5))
 (via (at 24.0603 41.9862) (size 0.6) (drill 0.3) (layers "F.Cu" "B.Cu") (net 5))
 (segment (start 56.83 42.45) (end 56.3662 41.9862) (width 0.2) (layer "B.Cu") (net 5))
 (segment (start 56.3662 41.9862) (end 24.0603 41.9862) (width 0.2) (layer "B.Cu") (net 5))
 (segment (start 16.8429 35.6005) (end 16.8429 35.6196) (width 0.2) (layer "F.Cu") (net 6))
 (segment (start 45.8374 43) (end 46.1683 43.3309) (width 0.2) (layer "F.Cu") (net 6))
 (segment (start 13.9517 40.9283) (end 16.8429 38.0371) (width 0.2) (layer "F.Cu") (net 6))
 (segment (start 47.42 44.65) (end 46.1683 44.65) (width 0.2) (layer "F.Cu") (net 6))
 (segment (start 16.8429 38.0371) (end 16.8429 35.6005) (width 0.2) (layer "F.Cu") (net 6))
 (segment (start 46.1683 43) (end 45.8374 43) (width 0.2) (layer "F.Cu") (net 6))
 (segment (start 46.1683 43.3309) (end 46.1683 44.65) (width 0.2) (layer "F.Cu") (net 6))
 (segment (start 13.15 41.73) (end 13.15 40.9283) (width 0.2) (layer "F.Cu") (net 6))
 (segment (start 13.15 40.9283) (end 13.9517 40.9283) (width 0.2) (layer "F.Cu") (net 6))
 (via (at 45.8374 43) (size 0.6) (drill 0.3) (layers "F.Cu" "B.Cu") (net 6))
 (via (at 16.8429 35.6005) (size 0.6) (drill 0.3) (layers "F.Cu" "B.Cu") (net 6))
 (segment (start 16.8429 35.6005) (end 16.8429 35.6196) (width 0.2) (layer "B.Cu") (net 6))
 (segment (start 46.1683 43) (end 45.8374 43) (width 0.2) (layer "B.Cu") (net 6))
 (segment (start 24.2233 43) (end 45.8374 43) (width 0.2) (layer "B.Cu") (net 6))
 (segment (start 16.8429 35.6196) (end 24.2233 43) (width 0.2) (layer "B.Cu") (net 6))
 (segment (start 16.45 44.27) (end 16.45 45.0717) (width 0.2) (layer "F.Cu") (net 3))
 (segment (start 34.67 39.4083) (end 34.67 17.71) (width 0.2) (layer "F.Cu") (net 3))
 (segment (start 33.53 40.9491) (end 33.53 40.5483) (width 0.2) (layer "F.Cu") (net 3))
 (segment (start 51.2502 10.4134) (end 52.5683 11.7315) (width 0.2) (layer "F.Cu") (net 3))
 (segment (start 16.45 45.0717) (end 16.4656 45.0873) (width 0.2) (layer "F.Cu") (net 3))
 (segment (start 40.9689 10.4134) (end 51.2502 10.4134) (width 0.2) (layer "F.Cu") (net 3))
 (segment (start 31.6959 40.9491) (end 33.53 40.9491) (width 0.2) (layer "F.Cu") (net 3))
 (segment (start 27.5577 45.0873) (end 31.6959 40.9491) (width 0.2) (layer "F.Cu") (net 3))
 (segment (start 33.53 40.5483) (end 34.67 39.4083) (width 0.2) (layer "F.Cu") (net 3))
 (segment (start 33.53 41.35) (end 33.53 40.9491) (width 0.2) (layer "F.Cu") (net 3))
 (segment (start 16.4656 45.0873) (end 27.5577 45.0873) (width 0.2) (layer "F.Cu") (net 3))
 (segment (start 39.7955 12.5845) (end 39.7955 11.5868) (width 0.2) (layer "F.Cu") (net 3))
 (segment (start 53.72 12) (end 52.5683 12) (width 0.2) (layer "F.Cu") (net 3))
 (segment (start 52.5683 11.7315) (end 52.5683 12) (width 0.2) (layer "F.Cu") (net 3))
 (segment (start 39.7955 11.5868) (end 40.9689 10.4134) (width 0.2) (layer "F.Cu") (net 3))
 (segment (start 34.67 17.71) (end 39.7955 12.5845) (width 0.2) (layer "F.Cu") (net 3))
 (segment (start 4.45 41.73) (end 4.45 42.5317) (width 0.2) (layer "F.Cu") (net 4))
 (segment (start 22.0883 35.1285) (end 22.0883 34.86) (width 0.2) (layer "F.Cu") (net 4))
 (segment (start 23.24 34.86) (end 22.0883 34.86) (width 0.2) (layer "F.Cu") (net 4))
 (segment (start 4.45 42.5317) (end 14.6851 42.5317) (width 0.2) (layer "F.Cu") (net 4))
 (segment (start 14.6851 42.5317) (end 22.0883 35.1285) (width 0.2) (layer "F.Cu") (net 4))
 (segment (start 42.2915 14.4202) (end 43.56 13.1517) (width 0.2) (layer "F.Cu") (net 2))
 (segment (start 30.99 44.65) (end 32.8635 44.65) (width 0.2) (layer "F.Cu") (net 2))
 (segment (start 43.56 12) (end 43.56 13.1517) (width 0.2) (layer "F.Cu") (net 2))
 (segment (start 32.8635 44.65) (end 42.2915 35.222) (width 0.2) (layer "F.Cu") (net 2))
 (segment (start 42.2915 35.222) (end 42.2915 14.4202) (width 0.2) (layer "F.Cu") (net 2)))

